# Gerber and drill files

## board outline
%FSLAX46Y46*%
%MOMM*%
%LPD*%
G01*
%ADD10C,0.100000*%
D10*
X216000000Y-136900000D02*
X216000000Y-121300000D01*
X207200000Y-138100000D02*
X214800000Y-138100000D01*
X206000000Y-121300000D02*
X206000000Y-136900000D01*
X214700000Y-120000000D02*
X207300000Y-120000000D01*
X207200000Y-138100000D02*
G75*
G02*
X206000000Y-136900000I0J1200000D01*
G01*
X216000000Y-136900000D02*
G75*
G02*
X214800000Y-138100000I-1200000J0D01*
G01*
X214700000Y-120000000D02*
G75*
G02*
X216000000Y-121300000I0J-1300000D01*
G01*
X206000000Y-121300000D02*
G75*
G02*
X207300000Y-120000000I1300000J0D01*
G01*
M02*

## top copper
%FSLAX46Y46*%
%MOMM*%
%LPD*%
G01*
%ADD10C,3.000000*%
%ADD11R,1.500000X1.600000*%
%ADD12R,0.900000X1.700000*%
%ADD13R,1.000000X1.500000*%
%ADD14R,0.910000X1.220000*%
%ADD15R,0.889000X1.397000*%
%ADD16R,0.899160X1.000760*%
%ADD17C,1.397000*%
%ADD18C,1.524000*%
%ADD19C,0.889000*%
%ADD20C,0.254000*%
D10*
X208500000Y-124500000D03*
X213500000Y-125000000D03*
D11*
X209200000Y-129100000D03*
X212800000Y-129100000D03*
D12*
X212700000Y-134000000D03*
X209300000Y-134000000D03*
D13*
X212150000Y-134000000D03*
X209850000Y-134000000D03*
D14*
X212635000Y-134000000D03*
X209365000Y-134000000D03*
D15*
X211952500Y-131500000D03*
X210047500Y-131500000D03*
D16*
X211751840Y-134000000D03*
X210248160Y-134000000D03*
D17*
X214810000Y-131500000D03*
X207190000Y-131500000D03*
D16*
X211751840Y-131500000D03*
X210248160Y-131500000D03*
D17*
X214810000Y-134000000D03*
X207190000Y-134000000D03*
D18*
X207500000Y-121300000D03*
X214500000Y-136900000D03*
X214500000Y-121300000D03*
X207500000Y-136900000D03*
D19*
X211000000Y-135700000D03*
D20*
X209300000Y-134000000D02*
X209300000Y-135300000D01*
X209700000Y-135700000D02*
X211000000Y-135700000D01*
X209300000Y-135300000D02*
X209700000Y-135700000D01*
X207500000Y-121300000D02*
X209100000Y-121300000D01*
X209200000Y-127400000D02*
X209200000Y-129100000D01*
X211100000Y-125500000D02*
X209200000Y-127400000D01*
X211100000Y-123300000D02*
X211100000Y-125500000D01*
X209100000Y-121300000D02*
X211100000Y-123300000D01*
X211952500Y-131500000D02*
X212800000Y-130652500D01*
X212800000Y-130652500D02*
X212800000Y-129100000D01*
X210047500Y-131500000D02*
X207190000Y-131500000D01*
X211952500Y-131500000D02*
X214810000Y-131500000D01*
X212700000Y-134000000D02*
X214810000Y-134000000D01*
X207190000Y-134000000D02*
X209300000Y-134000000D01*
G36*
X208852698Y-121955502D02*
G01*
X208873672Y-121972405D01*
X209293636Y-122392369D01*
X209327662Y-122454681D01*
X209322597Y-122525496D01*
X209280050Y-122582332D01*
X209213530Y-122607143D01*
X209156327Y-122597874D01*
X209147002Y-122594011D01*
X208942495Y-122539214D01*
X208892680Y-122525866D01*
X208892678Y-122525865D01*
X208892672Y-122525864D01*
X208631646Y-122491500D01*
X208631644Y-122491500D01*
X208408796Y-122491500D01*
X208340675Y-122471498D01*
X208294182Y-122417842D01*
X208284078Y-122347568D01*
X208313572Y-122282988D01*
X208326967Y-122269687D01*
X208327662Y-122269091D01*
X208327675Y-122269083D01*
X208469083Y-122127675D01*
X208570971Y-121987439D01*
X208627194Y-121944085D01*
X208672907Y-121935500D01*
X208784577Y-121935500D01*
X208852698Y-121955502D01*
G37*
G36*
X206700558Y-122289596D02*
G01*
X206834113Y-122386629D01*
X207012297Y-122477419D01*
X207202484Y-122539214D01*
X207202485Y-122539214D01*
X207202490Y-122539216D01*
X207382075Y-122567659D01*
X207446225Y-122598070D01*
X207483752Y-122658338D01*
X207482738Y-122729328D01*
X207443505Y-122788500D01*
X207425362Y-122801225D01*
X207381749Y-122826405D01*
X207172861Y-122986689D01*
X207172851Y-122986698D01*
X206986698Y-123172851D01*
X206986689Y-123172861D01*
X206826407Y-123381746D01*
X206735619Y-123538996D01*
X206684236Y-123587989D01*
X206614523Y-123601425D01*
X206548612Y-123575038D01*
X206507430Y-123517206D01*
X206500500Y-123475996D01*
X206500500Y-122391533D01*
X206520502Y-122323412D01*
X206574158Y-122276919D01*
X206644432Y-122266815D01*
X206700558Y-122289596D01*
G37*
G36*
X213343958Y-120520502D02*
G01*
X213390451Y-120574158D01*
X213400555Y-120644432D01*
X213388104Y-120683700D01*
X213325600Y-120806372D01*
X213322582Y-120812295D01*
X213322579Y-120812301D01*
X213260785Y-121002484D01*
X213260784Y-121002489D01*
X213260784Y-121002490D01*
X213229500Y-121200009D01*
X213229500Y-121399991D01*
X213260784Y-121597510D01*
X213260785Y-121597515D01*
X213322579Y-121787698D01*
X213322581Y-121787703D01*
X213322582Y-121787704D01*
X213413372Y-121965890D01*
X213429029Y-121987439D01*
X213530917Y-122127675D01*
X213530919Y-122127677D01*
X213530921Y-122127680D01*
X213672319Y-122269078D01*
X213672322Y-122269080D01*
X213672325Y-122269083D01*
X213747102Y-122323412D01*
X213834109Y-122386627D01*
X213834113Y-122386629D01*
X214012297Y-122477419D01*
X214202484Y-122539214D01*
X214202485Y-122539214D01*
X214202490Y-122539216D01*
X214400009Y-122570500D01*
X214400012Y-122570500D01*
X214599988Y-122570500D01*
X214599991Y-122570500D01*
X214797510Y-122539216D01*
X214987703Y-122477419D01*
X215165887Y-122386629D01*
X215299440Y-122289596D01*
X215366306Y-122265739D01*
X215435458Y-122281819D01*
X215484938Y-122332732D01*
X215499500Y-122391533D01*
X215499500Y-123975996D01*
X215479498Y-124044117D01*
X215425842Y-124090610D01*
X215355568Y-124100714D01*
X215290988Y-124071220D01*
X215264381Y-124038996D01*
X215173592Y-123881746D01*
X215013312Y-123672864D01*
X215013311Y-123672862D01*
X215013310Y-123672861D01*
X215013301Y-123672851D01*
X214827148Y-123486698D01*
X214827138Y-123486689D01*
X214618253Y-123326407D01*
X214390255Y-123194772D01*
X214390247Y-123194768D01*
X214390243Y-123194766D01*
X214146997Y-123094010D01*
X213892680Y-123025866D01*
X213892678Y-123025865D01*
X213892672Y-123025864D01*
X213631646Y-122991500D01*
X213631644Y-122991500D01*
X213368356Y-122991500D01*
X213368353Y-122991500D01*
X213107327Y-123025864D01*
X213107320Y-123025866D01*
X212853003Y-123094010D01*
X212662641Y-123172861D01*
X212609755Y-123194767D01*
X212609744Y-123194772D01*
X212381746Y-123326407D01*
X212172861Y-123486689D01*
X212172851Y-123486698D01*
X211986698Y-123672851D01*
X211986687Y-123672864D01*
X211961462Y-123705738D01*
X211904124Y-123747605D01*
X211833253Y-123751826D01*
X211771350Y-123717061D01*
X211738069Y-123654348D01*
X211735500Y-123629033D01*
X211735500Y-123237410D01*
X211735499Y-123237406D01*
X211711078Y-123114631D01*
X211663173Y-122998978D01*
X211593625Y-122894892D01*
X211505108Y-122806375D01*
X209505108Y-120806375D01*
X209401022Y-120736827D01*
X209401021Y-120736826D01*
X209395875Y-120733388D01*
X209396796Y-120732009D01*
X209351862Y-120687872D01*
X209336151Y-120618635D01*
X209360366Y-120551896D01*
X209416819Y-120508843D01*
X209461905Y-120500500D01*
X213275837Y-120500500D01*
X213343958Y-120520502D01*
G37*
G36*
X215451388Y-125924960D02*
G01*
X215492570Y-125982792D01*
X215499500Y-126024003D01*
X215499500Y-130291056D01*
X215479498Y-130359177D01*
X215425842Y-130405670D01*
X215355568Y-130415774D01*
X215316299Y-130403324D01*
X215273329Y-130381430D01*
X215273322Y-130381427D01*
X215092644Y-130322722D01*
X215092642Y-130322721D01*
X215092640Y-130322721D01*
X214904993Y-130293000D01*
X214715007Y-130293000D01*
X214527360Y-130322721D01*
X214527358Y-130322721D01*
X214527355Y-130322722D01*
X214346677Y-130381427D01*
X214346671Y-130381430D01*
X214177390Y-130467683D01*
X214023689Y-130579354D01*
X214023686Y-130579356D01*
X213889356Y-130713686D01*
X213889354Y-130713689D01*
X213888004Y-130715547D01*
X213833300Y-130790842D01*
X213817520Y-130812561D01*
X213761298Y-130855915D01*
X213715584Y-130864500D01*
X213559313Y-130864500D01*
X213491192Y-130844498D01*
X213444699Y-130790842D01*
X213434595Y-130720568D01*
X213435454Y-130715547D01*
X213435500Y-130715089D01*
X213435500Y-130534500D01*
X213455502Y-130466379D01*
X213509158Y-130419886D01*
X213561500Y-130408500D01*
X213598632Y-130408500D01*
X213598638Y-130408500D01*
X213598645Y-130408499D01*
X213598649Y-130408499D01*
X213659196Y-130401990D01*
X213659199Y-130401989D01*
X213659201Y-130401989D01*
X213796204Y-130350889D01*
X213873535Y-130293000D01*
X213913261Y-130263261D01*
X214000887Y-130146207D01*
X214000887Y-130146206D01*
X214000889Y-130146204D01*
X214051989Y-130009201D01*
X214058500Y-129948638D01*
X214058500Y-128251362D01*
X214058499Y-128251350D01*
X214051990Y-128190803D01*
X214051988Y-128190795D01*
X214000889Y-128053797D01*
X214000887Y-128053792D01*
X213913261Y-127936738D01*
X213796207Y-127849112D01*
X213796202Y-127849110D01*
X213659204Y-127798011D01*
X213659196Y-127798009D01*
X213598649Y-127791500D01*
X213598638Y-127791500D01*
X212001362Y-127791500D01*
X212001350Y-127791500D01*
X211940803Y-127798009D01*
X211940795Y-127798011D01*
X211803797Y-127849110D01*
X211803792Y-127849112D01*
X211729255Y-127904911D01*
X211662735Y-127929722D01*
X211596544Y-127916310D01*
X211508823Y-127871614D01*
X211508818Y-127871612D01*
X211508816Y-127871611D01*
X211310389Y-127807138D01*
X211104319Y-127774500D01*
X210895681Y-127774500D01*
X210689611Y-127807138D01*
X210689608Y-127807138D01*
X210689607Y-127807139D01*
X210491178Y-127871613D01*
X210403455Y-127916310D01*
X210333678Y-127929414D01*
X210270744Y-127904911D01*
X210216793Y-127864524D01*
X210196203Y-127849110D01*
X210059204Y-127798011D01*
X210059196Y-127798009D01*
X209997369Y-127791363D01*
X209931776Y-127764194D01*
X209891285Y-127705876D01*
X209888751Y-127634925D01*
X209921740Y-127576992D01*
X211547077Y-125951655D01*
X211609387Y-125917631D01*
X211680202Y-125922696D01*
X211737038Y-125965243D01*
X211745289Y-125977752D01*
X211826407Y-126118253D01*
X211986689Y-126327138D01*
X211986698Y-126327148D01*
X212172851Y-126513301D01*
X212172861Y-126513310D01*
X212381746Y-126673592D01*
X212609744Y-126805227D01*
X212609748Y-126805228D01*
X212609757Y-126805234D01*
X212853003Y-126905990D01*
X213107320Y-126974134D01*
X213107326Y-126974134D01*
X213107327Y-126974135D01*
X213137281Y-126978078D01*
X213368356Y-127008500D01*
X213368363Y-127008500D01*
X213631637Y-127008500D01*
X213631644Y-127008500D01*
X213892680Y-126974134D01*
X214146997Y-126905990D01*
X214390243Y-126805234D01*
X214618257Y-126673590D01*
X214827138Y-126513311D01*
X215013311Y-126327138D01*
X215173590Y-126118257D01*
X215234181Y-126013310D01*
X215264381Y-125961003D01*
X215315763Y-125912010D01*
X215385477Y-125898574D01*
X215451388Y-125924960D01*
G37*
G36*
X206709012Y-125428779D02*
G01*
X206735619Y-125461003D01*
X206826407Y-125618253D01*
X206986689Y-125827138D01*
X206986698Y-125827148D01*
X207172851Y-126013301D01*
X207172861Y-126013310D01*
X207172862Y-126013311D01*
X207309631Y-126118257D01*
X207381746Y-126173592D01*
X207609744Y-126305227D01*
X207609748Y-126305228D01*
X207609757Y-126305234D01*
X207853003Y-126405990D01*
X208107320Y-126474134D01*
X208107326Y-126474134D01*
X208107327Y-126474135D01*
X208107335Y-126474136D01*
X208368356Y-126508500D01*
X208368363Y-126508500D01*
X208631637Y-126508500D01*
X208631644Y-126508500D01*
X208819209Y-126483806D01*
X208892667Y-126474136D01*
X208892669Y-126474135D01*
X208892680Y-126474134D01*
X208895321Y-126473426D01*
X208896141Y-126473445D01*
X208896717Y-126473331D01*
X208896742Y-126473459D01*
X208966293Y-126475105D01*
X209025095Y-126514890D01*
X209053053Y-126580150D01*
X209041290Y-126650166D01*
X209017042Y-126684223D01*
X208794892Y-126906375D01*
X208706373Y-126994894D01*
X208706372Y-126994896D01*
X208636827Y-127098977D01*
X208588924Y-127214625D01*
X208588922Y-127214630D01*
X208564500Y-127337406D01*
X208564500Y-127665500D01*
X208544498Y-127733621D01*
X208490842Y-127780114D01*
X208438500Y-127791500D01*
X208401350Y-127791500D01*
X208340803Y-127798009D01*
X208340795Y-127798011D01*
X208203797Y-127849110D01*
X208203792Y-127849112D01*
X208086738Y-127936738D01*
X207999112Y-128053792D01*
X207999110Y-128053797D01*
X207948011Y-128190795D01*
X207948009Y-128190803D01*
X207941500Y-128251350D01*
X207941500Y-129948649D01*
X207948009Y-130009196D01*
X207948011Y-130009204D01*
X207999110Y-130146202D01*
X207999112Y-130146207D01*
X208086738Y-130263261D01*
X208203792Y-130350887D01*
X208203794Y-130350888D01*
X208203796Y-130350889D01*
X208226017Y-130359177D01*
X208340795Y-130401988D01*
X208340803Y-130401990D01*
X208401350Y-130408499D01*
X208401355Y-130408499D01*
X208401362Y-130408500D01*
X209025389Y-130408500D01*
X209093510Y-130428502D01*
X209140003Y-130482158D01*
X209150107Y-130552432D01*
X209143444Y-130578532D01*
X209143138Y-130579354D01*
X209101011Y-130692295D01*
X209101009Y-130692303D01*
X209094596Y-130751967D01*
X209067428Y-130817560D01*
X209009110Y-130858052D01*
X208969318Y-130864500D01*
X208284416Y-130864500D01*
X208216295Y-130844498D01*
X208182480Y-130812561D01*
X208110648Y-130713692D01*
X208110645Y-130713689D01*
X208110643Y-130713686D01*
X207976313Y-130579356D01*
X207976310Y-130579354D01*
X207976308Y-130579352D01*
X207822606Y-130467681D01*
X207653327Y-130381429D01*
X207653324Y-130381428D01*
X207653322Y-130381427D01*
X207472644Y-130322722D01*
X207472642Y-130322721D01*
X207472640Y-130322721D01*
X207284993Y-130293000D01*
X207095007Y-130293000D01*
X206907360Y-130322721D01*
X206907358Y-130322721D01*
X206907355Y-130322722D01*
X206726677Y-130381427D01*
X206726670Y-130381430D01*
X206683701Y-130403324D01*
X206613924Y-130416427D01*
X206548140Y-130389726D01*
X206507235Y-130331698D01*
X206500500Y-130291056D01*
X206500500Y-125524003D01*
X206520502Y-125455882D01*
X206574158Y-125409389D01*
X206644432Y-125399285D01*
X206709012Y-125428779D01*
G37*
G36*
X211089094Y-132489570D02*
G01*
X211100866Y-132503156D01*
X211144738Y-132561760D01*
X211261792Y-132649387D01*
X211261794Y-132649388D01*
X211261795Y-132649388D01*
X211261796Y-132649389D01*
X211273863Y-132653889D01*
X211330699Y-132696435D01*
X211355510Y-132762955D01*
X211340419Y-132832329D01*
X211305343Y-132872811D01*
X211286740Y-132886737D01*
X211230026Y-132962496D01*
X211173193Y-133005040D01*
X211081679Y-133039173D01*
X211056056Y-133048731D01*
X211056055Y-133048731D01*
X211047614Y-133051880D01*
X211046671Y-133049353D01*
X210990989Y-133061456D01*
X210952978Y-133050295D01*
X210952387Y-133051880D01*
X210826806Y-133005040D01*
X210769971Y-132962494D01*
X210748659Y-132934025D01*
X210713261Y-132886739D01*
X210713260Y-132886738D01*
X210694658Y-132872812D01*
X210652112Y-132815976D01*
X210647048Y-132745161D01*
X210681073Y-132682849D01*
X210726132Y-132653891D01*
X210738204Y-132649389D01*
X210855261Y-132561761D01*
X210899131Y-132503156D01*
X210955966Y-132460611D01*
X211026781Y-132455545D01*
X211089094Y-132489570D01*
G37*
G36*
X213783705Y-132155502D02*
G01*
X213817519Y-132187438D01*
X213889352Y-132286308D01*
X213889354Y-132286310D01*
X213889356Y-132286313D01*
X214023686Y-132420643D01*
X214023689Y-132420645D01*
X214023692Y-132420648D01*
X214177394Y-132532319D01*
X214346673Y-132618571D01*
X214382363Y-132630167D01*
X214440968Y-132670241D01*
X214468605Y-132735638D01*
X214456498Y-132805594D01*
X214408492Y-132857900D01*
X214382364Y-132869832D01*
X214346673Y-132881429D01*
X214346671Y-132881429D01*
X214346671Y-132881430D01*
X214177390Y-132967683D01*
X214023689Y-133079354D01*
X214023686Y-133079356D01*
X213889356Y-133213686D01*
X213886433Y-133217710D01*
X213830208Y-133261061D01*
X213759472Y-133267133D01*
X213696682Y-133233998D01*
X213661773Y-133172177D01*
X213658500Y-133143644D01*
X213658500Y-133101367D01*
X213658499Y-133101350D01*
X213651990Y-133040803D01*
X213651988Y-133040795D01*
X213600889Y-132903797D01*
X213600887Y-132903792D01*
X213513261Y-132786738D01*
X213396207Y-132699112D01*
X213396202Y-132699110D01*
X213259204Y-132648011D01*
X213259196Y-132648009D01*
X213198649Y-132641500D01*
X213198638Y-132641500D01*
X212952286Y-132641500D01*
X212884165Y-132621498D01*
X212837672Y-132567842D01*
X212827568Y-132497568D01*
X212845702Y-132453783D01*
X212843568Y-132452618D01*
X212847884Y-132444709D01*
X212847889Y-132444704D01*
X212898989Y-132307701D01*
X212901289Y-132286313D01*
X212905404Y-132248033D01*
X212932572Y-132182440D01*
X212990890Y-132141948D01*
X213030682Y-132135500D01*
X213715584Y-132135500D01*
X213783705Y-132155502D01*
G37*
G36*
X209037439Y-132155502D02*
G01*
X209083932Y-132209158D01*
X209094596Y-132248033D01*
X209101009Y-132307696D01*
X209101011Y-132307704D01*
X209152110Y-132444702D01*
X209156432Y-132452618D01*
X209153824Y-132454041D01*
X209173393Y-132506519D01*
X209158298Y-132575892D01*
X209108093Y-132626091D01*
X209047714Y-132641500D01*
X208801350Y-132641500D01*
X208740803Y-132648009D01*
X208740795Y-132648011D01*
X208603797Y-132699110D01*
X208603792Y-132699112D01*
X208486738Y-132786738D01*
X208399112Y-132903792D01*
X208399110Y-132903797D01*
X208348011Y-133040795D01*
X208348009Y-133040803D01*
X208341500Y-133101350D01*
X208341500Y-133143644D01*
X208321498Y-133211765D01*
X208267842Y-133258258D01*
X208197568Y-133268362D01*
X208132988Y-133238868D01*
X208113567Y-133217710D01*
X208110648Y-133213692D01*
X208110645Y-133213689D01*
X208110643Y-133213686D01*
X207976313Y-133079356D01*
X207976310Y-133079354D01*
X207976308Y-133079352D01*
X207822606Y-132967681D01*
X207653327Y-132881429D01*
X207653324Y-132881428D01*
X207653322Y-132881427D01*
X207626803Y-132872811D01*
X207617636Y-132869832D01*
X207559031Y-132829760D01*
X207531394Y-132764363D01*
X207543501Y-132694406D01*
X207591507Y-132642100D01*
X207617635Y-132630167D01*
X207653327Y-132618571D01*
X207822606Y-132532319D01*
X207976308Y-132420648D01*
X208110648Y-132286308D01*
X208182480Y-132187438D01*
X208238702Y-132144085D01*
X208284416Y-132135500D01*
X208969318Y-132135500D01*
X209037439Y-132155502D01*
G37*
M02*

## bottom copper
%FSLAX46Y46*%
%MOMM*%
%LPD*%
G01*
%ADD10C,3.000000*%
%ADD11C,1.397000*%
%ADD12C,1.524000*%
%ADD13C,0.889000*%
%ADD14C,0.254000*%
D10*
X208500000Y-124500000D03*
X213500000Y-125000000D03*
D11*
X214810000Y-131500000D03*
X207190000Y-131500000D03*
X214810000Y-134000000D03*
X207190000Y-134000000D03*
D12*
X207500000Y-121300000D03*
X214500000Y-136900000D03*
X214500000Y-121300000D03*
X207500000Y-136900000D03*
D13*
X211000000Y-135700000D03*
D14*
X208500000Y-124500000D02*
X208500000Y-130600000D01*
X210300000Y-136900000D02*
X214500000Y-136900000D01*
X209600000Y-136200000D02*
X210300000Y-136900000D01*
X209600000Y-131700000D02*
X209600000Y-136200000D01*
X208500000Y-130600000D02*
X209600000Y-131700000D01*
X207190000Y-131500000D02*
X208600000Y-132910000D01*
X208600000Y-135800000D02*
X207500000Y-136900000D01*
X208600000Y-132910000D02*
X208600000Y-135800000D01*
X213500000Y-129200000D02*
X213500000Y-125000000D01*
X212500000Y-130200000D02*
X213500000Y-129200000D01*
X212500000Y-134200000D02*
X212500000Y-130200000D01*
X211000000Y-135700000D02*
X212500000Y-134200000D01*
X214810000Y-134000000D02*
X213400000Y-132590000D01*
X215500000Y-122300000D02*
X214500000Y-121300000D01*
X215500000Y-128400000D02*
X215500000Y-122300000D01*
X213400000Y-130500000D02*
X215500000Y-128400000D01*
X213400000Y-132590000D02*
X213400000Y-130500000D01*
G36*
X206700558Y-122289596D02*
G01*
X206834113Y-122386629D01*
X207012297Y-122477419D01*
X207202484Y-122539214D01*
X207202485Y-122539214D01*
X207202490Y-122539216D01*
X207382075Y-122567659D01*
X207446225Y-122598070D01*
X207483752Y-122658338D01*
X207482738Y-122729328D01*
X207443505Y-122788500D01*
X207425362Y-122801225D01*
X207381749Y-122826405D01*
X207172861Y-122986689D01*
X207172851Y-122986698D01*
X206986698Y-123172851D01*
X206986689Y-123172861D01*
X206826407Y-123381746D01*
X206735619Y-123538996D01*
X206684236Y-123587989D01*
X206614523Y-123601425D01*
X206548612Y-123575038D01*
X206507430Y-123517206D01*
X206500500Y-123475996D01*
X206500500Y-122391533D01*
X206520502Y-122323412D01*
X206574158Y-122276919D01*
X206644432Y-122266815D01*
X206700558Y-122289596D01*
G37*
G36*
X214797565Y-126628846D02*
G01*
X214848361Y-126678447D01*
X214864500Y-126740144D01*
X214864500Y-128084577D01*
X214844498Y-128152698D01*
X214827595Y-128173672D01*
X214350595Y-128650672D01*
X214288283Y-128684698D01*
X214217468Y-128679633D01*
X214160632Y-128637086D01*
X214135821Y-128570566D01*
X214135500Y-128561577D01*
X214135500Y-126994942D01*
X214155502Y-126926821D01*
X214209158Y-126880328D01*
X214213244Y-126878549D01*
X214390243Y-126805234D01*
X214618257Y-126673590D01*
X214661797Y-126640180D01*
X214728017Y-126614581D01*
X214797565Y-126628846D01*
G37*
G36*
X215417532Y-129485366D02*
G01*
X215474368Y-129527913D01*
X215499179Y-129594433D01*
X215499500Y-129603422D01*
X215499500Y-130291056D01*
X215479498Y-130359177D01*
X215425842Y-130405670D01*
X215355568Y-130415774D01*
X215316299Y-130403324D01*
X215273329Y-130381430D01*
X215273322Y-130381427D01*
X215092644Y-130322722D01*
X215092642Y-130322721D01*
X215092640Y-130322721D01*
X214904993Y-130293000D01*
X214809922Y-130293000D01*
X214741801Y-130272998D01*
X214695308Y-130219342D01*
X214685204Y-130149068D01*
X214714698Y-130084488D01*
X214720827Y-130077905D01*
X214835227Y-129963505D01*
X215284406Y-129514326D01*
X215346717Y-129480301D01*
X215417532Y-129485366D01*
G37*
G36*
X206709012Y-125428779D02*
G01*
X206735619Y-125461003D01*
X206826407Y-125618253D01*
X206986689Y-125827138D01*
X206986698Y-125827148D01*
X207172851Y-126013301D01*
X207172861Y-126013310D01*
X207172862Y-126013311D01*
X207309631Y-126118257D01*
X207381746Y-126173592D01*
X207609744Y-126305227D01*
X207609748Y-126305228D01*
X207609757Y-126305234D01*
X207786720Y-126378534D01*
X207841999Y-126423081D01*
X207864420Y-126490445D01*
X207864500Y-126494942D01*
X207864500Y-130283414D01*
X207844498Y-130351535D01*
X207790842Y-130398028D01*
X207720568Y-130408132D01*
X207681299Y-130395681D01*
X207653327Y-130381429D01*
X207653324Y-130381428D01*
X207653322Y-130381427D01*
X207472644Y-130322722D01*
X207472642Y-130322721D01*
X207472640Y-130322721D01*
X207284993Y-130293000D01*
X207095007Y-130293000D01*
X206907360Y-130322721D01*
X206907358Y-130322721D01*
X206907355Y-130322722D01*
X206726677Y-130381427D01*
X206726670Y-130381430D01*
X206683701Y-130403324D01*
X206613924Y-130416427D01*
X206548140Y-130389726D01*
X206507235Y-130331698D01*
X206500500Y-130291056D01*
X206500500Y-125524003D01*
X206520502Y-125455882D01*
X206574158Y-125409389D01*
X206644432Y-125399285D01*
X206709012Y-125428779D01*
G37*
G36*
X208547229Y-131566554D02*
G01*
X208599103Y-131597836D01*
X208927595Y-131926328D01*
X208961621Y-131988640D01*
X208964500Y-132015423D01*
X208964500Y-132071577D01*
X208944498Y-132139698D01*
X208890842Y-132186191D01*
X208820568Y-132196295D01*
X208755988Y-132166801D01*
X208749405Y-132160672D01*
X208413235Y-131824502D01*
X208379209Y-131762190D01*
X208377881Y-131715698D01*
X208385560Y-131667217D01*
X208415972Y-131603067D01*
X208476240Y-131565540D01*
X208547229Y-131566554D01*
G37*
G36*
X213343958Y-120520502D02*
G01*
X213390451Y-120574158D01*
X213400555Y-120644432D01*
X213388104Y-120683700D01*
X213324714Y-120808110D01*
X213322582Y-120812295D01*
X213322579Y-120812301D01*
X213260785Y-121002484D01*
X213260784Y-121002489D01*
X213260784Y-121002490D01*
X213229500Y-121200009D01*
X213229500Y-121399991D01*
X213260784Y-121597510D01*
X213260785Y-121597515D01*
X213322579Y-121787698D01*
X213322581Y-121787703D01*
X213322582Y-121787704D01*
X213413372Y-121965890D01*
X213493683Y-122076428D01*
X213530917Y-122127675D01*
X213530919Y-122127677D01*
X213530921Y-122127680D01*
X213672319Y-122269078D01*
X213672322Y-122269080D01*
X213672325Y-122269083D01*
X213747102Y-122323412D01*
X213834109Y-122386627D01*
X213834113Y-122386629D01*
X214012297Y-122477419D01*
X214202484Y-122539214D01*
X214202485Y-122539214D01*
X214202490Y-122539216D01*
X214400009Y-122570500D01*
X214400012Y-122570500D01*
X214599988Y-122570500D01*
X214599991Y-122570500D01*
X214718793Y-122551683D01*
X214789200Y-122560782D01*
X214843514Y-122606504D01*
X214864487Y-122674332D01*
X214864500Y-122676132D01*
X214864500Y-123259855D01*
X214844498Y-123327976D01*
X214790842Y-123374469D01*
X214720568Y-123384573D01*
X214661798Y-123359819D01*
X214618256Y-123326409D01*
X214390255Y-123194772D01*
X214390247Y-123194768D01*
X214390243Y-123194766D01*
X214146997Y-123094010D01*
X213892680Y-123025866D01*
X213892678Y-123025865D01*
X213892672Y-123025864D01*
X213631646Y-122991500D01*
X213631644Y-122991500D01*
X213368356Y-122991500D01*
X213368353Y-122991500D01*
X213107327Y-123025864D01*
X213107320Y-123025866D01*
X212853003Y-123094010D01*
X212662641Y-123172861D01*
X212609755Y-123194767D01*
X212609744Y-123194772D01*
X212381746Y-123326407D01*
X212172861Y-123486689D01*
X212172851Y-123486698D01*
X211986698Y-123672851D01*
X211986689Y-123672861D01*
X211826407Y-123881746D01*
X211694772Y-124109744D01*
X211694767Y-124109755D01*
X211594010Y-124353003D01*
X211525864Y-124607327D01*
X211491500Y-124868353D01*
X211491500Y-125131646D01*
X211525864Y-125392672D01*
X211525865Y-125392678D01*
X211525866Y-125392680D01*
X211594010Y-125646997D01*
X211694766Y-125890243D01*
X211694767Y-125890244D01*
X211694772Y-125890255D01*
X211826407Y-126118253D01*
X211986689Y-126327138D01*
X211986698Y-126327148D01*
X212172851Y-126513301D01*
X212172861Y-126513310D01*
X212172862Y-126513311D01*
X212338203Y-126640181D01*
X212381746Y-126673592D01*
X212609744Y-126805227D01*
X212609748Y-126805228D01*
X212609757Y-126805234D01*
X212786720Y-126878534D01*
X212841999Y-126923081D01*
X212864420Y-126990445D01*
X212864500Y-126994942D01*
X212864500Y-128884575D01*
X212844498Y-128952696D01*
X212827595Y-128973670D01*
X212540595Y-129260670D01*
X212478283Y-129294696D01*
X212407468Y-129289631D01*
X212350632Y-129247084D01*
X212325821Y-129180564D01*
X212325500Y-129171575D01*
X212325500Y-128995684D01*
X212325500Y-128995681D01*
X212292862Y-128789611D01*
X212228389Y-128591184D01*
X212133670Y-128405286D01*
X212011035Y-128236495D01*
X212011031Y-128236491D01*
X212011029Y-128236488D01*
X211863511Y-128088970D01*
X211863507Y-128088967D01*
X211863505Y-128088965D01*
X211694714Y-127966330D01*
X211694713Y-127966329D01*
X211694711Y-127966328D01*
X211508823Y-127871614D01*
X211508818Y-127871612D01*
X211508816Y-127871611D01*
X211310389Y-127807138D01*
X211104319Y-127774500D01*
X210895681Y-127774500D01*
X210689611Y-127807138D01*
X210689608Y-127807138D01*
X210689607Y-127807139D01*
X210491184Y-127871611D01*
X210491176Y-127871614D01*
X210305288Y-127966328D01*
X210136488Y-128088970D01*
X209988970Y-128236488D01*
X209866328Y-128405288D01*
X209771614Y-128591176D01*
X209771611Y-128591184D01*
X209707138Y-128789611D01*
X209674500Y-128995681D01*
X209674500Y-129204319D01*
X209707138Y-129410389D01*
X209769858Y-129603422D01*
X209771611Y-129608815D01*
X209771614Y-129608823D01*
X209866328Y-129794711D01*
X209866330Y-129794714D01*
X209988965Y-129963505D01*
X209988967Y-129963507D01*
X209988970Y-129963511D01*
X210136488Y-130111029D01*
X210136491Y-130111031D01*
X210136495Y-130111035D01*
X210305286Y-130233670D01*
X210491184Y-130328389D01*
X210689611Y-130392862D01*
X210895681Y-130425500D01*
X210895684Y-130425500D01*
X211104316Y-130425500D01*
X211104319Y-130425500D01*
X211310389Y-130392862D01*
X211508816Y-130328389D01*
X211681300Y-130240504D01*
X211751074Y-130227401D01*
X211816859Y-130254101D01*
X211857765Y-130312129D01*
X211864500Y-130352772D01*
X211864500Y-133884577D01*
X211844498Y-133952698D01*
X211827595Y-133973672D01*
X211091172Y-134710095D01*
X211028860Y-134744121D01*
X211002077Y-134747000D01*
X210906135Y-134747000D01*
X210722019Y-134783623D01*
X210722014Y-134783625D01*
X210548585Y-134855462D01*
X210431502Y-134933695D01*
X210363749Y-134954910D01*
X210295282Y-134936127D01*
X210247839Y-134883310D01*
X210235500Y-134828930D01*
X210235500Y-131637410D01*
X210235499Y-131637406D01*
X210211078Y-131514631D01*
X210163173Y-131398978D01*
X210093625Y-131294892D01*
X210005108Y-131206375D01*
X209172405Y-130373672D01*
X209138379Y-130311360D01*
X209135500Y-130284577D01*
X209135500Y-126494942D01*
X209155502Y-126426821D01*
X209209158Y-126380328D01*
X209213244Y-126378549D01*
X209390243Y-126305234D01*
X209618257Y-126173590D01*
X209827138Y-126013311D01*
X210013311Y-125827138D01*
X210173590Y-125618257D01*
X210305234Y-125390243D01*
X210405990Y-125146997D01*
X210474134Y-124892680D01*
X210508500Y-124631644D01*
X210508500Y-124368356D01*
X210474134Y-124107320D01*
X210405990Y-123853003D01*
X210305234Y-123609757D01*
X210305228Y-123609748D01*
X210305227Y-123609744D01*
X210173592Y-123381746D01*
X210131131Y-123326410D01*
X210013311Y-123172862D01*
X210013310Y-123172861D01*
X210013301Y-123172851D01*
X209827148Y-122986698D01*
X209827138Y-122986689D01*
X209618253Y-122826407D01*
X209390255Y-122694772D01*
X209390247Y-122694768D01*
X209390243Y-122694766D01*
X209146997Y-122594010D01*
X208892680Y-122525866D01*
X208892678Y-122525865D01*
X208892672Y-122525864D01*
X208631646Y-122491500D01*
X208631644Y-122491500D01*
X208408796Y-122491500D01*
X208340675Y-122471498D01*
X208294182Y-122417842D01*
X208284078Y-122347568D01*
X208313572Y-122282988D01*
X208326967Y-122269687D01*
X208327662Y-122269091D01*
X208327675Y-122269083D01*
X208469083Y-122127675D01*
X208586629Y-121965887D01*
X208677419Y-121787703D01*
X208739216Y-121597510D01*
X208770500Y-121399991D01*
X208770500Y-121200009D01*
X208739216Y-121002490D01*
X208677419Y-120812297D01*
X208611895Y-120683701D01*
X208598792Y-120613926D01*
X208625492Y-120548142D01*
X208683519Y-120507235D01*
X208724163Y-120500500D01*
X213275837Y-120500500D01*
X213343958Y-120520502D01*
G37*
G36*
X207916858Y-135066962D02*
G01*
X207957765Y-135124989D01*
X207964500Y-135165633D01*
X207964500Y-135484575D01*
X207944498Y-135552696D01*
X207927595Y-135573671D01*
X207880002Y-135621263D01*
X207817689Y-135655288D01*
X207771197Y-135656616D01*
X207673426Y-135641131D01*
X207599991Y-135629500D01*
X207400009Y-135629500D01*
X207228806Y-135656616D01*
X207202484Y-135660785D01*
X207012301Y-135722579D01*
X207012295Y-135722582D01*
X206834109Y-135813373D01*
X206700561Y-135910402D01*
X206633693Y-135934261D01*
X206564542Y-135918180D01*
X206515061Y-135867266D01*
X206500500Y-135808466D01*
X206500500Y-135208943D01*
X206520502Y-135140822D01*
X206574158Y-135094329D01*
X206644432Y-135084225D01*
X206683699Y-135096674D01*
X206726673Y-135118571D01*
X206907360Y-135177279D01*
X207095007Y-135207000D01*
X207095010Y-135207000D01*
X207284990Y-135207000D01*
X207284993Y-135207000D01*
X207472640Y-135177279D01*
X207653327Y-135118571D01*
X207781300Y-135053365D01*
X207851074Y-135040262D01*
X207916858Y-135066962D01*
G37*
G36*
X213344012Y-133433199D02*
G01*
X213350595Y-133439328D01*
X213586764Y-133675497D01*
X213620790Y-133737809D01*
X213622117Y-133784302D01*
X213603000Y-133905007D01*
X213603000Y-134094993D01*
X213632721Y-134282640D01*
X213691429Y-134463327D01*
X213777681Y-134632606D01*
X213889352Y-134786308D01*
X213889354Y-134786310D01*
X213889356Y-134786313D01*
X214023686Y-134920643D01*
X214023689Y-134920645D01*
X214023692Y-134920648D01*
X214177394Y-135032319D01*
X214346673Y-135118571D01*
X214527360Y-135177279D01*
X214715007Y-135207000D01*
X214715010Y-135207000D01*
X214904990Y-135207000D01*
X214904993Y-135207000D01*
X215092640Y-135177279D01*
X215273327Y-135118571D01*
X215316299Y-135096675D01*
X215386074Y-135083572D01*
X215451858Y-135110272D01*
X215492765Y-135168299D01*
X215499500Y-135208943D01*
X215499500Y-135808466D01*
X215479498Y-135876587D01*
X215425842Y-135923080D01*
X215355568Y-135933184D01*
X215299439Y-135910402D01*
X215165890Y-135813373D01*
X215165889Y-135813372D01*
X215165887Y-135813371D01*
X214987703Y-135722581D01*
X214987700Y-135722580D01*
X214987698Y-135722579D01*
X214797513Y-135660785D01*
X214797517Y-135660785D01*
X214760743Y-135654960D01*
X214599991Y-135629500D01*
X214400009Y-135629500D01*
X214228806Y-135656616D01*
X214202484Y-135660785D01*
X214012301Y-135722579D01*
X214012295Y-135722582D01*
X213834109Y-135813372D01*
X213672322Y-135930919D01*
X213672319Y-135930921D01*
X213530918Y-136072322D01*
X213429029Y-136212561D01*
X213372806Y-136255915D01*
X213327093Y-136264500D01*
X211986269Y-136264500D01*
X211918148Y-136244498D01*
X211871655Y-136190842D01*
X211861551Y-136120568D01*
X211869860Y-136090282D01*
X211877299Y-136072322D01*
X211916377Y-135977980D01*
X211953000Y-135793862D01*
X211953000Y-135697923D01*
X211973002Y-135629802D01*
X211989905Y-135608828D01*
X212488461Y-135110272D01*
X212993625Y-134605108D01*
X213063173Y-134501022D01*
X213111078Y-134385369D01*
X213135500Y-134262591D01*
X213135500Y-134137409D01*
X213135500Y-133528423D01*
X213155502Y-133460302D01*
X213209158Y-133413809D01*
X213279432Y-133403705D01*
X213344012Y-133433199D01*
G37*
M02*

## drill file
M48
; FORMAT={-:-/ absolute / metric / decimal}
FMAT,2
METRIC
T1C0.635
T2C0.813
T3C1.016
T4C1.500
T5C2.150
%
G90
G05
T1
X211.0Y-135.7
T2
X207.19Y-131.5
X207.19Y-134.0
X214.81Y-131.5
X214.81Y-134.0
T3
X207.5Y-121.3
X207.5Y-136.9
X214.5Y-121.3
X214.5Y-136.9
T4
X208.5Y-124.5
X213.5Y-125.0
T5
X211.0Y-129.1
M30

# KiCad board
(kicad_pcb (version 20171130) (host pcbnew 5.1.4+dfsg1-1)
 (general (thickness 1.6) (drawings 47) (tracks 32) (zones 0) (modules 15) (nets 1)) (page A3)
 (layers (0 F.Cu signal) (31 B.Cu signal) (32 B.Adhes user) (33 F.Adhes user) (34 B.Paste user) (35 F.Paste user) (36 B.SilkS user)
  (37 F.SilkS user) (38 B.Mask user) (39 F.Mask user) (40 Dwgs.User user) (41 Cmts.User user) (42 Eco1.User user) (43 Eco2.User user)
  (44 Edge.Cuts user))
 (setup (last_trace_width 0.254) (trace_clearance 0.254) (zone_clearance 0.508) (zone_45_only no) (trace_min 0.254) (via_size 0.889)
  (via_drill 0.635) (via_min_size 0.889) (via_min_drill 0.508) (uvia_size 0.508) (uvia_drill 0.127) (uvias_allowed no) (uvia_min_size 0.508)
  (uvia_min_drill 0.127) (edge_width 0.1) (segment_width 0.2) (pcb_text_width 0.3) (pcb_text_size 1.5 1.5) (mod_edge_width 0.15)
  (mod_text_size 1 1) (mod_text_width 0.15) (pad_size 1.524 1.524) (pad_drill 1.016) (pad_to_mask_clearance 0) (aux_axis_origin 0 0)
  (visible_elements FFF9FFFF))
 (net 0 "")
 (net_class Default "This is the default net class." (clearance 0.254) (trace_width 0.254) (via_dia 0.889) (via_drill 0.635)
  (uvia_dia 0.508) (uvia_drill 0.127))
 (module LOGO (layer F.Cu) (at 211.1 122.9)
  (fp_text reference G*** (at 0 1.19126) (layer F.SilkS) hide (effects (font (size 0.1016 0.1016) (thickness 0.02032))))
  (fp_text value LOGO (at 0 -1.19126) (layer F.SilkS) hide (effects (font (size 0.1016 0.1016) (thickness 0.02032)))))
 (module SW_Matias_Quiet (layer F.Cu) (at 211 129)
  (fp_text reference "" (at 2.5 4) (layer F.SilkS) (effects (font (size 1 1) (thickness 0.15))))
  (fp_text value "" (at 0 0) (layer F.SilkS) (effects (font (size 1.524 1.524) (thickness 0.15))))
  (pad 1 thru_hole circle (at -2.5 -4.5) (size 3 3) (drill 1.5) (layers *.Cu *.Mask F.SilkS))
  (pad 2 thru_hole circle (at 2.5 -4) (size 3 3) (drill 1.5) (layers *.Cu *.Mask F.SilkS)))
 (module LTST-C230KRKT (layer F.Cu) (at 211 129.1)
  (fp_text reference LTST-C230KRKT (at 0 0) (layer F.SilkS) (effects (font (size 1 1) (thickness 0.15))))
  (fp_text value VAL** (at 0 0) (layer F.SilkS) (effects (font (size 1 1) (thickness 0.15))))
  (pad 2 smd rect (at -1.8 0) (size 1.5 1.6) (layers F.Cu F.Paste F.Mask))
  (pad 3 smd rect (at 1.8 0) (size 1.5 1.6) (layers F.Cu F.Paste F.Mask))
  (pad "" np_thru_hole circle (at 0 0) (size 2.15 2.15) (drill 2.15) (layers *.Cu *.Mask F.SilkS)))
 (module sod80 (layer F.Cu) (at 211 134)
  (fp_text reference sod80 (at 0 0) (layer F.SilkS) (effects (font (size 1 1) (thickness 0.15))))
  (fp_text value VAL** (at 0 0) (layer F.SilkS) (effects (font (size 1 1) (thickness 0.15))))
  (pad 5 smd rect (at 1.7 0) (size 0.9 1.7) (layers F.Cu F.Paste F.Mask))
  (pad 6 smd rect (at -1.7 0) (size 0.9 1.7) (layers F.Cu F.Paste F.Mask)))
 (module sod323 (layer F.Cu) (at 211 134)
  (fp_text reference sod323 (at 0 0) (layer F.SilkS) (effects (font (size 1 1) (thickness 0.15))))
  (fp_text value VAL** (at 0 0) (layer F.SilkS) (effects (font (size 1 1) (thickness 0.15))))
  (pad 3 smd rect (at 1.15 0) (size 1 1.5) (layers F.Cu F.Paste F.Mask))
  (pad 4 smd rect (at -1.15 0) (size 1 1.5) (layers F.Cu F.Paste F.Mask)))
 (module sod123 (layer F.Cu) (at 211 134)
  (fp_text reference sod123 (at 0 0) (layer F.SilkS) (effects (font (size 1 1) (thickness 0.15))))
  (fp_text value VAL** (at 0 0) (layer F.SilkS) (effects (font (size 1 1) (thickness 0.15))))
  (pad 1 smd rect (at 1.635 0) (size 0.91 1.22) (layers F.Cu F.Paste F.Mask))
  (pad 2 smd rect (at -1.635 0) (size 0.91 1.22) (layers F.Cu F.Paste F.Mask)))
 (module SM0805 (layer F.Cu) (at 211 131.5 180)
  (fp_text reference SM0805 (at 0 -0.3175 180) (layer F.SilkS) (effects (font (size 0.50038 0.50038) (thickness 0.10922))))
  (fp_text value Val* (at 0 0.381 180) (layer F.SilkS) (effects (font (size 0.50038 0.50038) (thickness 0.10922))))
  (pad 1 smd rect (at -0.9525 0 180) (size 0.889 1.397) (layers F.Cu F.Paste F.Mask))
  (pad 2 smd rect (at 0.9525 0 180) (size 0.889 1.397) (layers F.Cu F.Paste F.Mask)))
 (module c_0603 (layer F.Cu) (at 211 134)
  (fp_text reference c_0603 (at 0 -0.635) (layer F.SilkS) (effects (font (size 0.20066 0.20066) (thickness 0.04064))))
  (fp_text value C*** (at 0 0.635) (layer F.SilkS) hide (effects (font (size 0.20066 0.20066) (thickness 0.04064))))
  (pad 1 smd rect (at 0.75184 0) (size 0.89916 1.00076) (layers F.Cu F.Paste F.Mask))
  (pad 2 smd rect (at -0.75184 0) (size 0.89916 1.00076) (layers F.Cu F.Paste F.Mask)))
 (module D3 (layer F.Cu) (at 211 131.5)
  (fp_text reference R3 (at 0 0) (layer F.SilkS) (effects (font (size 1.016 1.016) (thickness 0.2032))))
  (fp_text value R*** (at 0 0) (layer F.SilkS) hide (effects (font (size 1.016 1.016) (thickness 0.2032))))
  (pad 2 thru_hole circle (at 3.81 0) (size 1.397 1.397) (drill 0.8128) (layers *.Cu *.Mask F.SilkS))
  (pad 1 thru_hole circle (at -3.81 0) (size 1.397 1.397) (drill 0.8128) (layers *.Cu *.Mask F.SilkS)))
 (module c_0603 (layer F.Cu) (at 211 131.5)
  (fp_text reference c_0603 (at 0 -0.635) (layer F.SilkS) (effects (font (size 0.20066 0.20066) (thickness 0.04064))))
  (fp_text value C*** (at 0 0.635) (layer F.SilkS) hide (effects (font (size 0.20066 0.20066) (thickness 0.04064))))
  (pad 1 smd rect (at 0.75184 0) (size 0.89916 1.00076) (layers F.Cu F.Paste F.Mask))
  (pad 2 smd rect (at -0.75184 0) (size 0.89916 1.00076) (layers F.Cu F.Paste F.Mask)))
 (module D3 (layer F.Cu) (at 211 134)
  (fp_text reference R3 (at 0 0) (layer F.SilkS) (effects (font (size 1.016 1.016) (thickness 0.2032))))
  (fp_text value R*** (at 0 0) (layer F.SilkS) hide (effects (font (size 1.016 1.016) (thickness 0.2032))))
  (pad 2 thru_hole circle (at 3.81 0) (size 1.397 1.397) (drill 0.8128) (layers *.Cu *.Mask F.SilkS))
  (pad 1 thru_hole circle (at -3.81 0) (size 1.397 1.397) (drill 0.8128) (layers *.Cu *.Mask F.SilkS)))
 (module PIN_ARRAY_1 (layer F.Cu) (at 207.5 121.3)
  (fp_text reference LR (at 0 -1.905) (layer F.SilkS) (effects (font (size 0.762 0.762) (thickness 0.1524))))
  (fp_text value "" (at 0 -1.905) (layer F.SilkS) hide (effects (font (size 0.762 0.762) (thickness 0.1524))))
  (pad 1 thru_hole circle (at 0 0) (size 1.524 1.524) (drill 1.016) (layers *.Cu *.Mask F.SilkS)))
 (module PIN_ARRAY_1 (layer F.Cu) (at 214.5 136.9)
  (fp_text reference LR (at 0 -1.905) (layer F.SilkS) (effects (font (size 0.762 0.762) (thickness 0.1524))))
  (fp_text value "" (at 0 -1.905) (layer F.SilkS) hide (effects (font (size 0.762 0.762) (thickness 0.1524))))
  (pad 1 thru_hole circle (at 0 0) (size 1.524 1.524) (drill 1.016) (layers *.Cu *.Mask F.SilkS)))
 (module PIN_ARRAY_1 (layer F.Cu) (at 214.5 121.3)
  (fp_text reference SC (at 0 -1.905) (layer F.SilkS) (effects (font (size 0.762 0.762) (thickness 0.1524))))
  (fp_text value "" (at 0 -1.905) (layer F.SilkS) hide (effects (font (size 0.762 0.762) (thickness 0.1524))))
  (pad 1 thru_hole circle (at 0 0) (size 1.524 1.524) (drill 1.016) (layers *.Cu *.Mask F.SilkS)))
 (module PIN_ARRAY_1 (layer F.Cu) (at 207.5 136.9)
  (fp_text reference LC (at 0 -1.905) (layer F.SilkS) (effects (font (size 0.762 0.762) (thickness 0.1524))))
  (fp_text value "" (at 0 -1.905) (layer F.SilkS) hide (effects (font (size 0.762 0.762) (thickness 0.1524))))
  (pad 1 thru_hole circle (at 0 0) (size 1.524 1.524) (drill 1.016) (layers *.Cu *.Mask F.SilkS)))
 (gr_line (start 216 136.9) (end 216 121.3) (angle 90) (layer Edge.Cuts) (width 0.1))
 (gr_line (start 207.2 138.1) (end 214.8 138.1) (angle 90) (layer Edge.Cuts) (width 0.1))
 (gr_line (start 206 121.3) (end 206 136.9) (angle 90) (layer Edge.Cuts) (width 0.1))
 (gr_line (start 214.7 120) (end 207.3 120) (angle 90) (layer Edge.Cuts) (width 0.1))
 (gr_arc (start 207.2 136.9) (end 207.2 138.1) (angle 90) (layer Edge.Cuts) (width 0.1))
 (gr_arc (start 214.8 136.9) (end 216 136.9) (angle 90) (layer Edge.Cuts) (width 0.1))
 (gr_arc (start 214.7 121.3) (end 214.7 120) (angle 90) (layer Edge.Cuts) (width 0.1))
 (gr_arc (start 207.3 121.3) (end 206 121.3) (angle 90) (layer Edge.Cuts) (width 0.1))
 (segment (start 208.5 124.5) (end 208.5 130.6) (width 0.254) (layer B.Cu) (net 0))
 (segment (start 210.3 136.9) (end 214.5 136.9) (width 0.254) (layer B.Cu) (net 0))
 (segment (start 209.6 136.2) (end 210.3 136.9) (width 0.254) (layer B.Cu) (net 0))
 (segment (start 209.6 131.7) (end 209.6 136.2) (width 0.254) (layer B.Cu) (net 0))
 (segment (start 208.5 130.6) (end 209.6 131.7) (width 0.254) (layer B.Cu) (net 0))
 (segment (start 207.19 131.5) (end 208.6 132.91) (width 0.254) (layer B.Cu) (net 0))
 (segment (start 208.6 135.8) (end 207.5 136.9) (width 0.254) (layer B.Cu) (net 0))
 (segment (start 208.6 132.91) (end 208.6 135.8) (width 0.254) (layer B.Cu) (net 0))
 (segment (start 209.3 134) (end 209.3 135.3) (width 0.254) (layer F.Cu) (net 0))
 (segment (start 213.5 129.2) (end 213.5 125) (width 0.254) (layer B.Cu) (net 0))
 (segment (start 212.5 130.2) (end 213.5 129.2) (width 0.254) (layer B.Cu) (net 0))
 (segment (start 212.5 134.2) (end 212.5 130.2) (width 0.254) (layer B.Cu) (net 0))
 (segment (start 211 135.7) (end 212.5 134.2) (width 0.254) (layer B.Cu) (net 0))
 (via (at 211 135.7) (size 0.889) (layers F.Cu B.Cu) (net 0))
 (segment (start 209.7 135.7) (end 211 135.7) (width 0.254) (layer F.Cu) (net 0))
 (segment (start 209.3 135.3) (end 209.7 135.7) (width 0.254) (layer F.Cu) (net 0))
 (segment (start 207.5 121.3) (end 209.1 121.3) (width 0.254) (layer F.Cu) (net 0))
 (segment (start 209.2 127.4) (end 209.2 129.1) (width 0.254) (layer F.Cu) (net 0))
 (segment (start 211.1 125.5) (end 209.2 127.4) (width 0.254) (layer F.Cu) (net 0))
 (segment (start 211.1 123.3) (end 211.1 125.5) (width 0.254) (layer F.Cu) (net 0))
 (segment (start 209.1 121.3) (end 211.1 123.3) (width 0.254) (layer F.Cu) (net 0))
 (segment (start 214.81 134) (end 213.4 132.59) (width 0.254) (layer B.Cu) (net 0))
 (segment (start 215.5 122.3) (end 214.5 121.3) (width 0.254) (layer B.Cu) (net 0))
 (segment (start 215.5 128.4) (end 215.5 122.3) (width 0.254) (layer B.Cu) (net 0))
 (segment (start 213.4 130.5) (end 215.5 128.4) (width 0.254) (layer B.Cu) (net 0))
 (segment (start 213.4 132.59) (end 213.4 130.5) (width 0.254) (layer B.Cu) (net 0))
 (segment (start 211.9525 131.5) (end 212.8 130.6525) (width 0.254) (layer F.Cu) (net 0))
 (segment (start 212.8 130.6525) (end 212.8 129.1) (width 0.254) (layer F.Cu) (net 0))
 (segment (start 210.0475 131.5) (end 207.19 131.5) (width 0.254) (layer F.Cu) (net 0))
 (segment (start 211.9525 131.5) (end 214.81 131.5) (width 0.254) (layer F.Cu) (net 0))
 (segment (start 212.7 134) (end 214.81 134) (width 0.254) (layer F.Cu) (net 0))
 (segment (start 207.19 134) (end 209.3 134) (width 0.254) (layer F.Cu) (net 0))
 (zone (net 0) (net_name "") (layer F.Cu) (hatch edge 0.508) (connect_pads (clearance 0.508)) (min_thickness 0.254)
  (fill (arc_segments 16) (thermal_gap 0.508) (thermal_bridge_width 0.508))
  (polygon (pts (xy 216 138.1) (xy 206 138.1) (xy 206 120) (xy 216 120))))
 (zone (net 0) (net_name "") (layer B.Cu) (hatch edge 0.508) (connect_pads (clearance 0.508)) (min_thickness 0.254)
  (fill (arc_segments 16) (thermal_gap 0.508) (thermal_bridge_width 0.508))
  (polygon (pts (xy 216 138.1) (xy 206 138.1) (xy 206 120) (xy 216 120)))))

